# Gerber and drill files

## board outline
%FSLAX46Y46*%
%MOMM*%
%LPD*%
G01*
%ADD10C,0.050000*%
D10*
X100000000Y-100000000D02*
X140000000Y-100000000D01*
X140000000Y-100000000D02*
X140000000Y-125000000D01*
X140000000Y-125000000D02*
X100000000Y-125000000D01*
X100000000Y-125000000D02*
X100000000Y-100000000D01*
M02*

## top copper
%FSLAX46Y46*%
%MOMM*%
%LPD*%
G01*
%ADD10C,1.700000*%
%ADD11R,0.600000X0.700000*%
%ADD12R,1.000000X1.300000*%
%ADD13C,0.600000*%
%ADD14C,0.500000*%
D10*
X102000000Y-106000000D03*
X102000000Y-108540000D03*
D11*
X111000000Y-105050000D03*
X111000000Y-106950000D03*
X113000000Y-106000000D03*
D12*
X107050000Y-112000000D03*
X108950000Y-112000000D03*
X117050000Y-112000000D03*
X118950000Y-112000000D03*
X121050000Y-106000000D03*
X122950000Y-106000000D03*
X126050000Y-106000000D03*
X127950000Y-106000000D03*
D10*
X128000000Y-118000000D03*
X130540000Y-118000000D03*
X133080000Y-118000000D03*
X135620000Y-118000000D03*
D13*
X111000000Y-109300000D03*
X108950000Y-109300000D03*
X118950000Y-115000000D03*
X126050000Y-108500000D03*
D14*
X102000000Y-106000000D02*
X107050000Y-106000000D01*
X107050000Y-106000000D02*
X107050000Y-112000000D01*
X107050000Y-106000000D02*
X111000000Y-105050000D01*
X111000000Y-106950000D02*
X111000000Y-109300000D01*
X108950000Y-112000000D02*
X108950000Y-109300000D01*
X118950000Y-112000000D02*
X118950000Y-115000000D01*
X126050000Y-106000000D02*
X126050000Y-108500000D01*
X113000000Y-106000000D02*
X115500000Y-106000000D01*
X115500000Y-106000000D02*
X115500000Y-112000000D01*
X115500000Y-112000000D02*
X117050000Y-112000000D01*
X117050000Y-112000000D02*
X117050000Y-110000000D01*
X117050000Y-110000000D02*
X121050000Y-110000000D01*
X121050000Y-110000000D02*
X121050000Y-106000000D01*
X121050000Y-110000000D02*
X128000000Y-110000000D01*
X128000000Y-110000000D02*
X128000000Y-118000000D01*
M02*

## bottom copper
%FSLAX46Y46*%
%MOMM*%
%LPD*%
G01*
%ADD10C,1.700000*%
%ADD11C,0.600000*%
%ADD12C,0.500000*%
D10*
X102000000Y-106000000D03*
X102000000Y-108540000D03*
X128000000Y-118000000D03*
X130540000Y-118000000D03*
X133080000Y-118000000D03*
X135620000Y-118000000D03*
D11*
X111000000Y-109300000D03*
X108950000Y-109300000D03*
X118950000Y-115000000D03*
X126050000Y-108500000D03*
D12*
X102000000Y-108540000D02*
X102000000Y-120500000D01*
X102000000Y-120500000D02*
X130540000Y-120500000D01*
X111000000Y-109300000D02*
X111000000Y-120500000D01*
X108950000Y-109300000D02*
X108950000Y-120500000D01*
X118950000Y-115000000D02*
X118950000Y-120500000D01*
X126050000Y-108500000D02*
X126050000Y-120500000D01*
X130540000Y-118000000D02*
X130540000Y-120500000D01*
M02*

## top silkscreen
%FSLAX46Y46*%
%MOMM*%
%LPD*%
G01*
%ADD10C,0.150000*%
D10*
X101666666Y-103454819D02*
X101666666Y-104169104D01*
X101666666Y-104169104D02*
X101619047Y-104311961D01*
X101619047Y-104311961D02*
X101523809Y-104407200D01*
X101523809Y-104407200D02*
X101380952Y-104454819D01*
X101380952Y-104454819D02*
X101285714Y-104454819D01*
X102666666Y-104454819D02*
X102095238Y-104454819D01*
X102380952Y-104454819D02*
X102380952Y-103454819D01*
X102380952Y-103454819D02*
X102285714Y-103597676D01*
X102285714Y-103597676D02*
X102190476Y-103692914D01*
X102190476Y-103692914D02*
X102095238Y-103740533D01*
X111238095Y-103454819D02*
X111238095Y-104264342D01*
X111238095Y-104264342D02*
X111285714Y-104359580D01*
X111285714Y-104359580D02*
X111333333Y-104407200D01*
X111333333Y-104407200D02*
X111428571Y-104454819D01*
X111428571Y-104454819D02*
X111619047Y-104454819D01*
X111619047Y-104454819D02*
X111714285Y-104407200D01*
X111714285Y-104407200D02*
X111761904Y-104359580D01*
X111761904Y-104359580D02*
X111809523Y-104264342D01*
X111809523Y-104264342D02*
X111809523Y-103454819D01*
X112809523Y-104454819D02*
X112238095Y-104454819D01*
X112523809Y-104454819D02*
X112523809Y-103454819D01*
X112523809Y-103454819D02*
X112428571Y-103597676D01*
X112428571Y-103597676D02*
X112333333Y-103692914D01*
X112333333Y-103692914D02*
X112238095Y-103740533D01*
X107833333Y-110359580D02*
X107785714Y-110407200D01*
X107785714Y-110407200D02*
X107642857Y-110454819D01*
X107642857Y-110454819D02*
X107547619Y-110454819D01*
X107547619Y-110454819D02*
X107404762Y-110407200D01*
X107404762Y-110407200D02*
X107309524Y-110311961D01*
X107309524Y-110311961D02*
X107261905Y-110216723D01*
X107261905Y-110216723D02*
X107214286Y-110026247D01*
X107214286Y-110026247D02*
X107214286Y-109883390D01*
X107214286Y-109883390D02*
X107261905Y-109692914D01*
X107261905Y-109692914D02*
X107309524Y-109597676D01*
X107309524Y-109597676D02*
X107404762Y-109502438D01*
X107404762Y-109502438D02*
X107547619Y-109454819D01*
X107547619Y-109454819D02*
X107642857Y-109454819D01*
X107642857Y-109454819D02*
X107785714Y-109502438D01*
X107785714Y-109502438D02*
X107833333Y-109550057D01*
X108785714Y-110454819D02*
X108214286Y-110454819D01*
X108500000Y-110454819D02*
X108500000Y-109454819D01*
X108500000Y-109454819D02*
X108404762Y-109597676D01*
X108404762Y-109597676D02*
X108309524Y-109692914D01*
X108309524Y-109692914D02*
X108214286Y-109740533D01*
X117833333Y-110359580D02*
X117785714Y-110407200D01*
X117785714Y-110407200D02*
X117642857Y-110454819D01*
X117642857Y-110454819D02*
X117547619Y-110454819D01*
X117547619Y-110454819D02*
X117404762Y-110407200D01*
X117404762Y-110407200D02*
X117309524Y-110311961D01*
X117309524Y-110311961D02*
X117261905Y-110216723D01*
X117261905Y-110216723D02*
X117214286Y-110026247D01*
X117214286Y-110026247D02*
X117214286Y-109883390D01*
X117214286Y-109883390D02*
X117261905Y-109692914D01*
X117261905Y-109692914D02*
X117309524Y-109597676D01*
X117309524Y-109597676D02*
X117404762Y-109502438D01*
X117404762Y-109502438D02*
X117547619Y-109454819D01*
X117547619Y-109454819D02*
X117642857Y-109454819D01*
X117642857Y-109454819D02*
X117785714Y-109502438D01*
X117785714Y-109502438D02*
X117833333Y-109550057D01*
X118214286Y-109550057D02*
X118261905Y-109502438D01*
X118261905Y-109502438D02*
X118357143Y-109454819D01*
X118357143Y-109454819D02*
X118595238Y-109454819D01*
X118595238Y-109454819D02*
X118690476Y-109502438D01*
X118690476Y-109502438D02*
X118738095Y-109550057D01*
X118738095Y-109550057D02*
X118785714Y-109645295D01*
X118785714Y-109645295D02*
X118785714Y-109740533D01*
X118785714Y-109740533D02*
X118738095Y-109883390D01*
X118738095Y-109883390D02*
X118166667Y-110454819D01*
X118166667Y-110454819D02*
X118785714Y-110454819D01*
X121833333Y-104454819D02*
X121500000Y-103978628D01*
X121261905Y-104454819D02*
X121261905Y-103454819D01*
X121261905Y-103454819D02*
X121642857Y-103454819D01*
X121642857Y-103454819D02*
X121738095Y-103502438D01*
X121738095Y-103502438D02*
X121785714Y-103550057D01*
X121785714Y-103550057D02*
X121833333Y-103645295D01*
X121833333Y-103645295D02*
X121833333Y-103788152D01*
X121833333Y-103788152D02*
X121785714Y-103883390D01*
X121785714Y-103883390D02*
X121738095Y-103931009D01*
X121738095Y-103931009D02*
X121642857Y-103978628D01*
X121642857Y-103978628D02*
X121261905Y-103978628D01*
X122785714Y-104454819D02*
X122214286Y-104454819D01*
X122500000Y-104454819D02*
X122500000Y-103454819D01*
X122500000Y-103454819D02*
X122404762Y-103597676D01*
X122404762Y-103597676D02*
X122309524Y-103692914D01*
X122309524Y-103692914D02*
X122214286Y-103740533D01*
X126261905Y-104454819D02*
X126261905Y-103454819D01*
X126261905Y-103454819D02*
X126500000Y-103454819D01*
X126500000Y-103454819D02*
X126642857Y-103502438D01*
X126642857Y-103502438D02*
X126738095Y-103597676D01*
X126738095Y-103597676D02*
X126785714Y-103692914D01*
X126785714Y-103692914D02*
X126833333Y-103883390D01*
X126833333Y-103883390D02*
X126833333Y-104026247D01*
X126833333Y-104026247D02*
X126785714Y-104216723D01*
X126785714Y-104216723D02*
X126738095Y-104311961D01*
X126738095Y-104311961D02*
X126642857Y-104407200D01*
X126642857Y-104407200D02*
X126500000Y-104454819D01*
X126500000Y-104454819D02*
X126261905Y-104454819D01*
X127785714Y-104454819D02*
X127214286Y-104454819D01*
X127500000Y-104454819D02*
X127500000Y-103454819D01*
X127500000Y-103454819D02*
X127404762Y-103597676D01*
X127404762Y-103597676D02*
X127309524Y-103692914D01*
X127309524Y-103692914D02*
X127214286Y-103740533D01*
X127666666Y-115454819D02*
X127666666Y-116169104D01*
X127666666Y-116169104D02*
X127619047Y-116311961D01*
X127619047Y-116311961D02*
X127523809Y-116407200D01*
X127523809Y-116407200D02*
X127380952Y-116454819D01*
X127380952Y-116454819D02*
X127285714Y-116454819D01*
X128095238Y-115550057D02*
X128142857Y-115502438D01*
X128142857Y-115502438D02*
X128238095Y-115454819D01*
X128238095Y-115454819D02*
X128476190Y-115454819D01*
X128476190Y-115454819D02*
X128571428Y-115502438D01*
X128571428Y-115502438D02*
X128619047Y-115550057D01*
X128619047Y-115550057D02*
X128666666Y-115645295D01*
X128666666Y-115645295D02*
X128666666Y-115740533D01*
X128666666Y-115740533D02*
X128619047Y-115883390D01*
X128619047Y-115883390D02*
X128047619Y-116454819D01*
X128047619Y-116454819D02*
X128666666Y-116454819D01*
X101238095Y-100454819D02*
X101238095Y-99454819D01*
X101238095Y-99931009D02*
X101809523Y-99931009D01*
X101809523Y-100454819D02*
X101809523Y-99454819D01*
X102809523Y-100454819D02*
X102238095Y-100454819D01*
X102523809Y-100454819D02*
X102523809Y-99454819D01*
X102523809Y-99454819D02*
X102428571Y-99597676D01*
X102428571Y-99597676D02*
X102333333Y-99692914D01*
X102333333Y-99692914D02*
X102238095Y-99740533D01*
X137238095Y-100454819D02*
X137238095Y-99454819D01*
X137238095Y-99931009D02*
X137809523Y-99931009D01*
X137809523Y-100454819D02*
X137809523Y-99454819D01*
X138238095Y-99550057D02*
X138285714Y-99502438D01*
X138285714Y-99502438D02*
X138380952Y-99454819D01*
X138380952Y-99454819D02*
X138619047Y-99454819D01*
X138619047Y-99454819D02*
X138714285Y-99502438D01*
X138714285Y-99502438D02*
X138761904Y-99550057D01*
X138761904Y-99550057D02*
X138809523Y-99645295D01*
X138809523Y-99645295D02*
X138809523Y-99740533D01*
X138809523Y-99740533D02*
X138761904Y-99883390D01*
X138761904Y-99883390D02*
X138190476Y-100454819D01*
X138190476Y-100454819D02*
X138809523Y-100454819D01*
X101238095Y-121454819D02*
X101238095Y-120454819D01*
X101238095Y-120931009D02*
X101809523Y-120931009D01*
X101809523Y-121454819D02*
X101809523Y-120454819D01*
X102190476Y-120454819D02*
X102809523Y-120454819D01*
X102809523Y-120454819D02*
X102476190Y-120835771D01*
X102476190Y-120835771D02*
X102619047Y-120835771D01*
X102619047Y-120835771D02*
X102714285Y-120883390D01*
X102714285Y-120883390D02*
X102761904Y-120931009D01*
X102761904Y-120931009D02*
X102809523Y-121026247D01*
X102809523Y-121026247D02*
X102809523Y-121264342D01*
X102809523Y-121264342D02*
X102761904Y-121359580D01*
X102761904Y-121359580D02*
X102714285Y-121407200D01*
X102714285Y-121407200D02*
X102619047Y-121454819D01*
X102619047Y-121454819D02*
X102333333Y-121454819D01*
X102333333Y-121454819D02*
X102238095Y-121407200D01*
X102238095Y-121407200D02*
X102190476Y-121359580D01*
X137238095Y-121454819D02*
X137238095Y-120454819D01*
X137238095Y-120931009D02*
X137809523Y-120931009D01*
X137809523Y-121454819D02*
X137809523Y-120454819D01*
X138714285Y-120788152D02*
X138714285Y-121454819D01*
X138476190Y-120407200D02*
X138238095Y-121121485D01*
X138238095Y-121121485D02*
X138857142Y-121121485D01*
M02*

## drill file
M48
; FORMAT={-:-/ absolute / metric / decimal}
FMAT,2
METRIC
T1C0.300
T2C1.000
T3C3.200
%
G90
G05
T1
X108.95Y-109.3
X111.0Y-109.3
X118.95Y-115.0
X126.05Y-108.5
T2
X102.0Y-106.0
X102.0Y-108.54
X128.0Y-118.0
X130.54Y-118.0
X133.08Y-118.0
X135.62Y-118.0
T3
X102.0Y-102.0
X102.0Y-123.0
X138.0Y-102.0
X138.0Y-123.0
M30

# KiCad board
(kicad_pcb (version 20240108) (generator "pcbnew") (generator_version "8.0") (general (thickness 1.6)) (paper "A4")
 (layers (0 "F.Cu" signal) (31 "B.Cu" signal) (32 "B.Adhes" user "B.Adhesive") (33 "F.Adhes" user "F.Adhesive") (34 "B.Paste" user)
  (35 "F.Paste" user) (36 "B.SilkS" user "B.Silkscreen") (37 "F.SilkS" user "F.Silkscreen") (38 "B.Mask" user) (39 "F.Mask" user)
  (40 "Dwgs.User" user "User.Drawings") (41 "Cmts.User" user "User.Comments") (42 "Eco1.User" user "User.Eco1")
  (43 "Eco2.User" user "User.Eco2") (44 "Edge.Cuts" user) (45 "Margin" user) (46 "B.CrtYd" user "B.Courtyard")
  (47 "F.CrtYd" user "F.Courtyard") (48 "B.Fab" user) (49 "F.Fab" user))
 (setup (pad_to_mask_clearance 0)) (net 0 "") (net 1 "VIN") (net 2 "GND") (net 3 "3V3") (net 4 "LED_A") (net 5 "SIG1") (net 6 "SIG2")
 (gr_line (start 100 100) (end 140 100) (stroke (width 0.05) (type default)) (layer "Edge.Cuts"))
 (gr_line (start 140 100) (end 140 125) (stroke (width 0.05) (type default)) (layer "Edge.Cuts"))
 (gr_line (start 140 125) (end 100 125) (stroke (width 0.05) (type default)) (layer "Edge.Cuts"))
 (gr_line (start 100 125) (end 100 100) (stroke (width 0.05) (type default)) (layer "Edge.Cuts"))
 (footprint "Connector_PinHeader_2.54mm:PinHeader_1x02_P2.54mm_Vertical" (layer "F.Cu") (at 102 106)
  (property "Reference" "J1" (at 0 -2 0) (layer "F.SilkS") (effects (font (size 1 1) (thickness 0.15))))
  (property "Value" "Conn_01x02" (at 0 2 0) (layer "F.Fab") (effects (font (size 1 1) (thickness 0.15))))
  (pad "1" thru_hole circle (at 0 0) (size 1.7 1.7) (drill 1) (layers "*.Cu" "*.Mask") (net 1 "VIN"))
  (pad "2" thru_hole circle (at 0 2.54) (size 1.7 1.7) (drill 1) (layers "*.Cu" "*.Mask") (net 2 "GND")))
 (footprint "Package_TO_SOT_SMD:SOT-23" (layer "F.Cu") (at 112 106)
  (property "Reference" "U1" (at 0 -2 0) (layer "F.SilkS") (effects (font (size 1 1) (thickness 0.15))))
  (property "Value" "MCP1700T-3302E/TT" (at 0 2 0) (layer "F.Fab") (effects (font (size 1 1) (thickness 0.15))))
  (pad "1" smd rect (at -1 -0.95) (size 0.6 0.7) (layers "F.Cu" "F.Paste" "F.Mask") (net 1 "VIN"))
  (pad "2" smd rect (at -1 0.95) (size 0.6 0.7) (layers "F.Cu" "F.Paste" "F.Mask") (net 2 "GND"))
  (pad "3" smd rect (at 1 0) (size 0.6 0.7) (layers "F.Cu" "F.Paste" "F.Mask") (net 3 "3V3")))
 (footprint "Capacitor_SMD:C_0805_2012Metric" (layer "F.Cu") (at 108 112)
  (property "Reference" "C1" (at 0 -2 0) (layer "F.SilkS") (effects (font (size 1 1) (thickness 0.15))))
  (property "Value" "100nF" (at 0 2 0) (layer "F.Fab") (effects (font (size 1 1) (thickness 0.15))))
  (pad "1" smd rect (at -0.95 0) (size 1 1.3) (layers "F.Cu" "F.Paste" "F.Mask") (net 1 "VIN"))
  (pad "2" smd rect (at 0.95 0) (size 1 1.3) (layers "F.Cu" "F.Paste" "F.Mask") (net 2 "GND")))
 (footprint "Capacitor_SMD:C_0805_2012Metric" (layer "F.Cu") (at 118 112)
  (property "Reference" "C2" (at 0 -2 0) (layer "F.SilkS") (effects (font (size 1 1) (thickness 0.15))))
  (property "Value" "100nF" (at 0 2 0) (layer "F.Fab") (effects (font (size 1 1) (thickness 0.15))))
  (pad "1" smd rect (at -0.95 0) (size 1 1.3) (layers "F.Cu" "F.Paste" "F.Mask") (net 3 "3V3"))
  (pad "2" smd rect (at 0.95 0) (size 1 1.3) (layers "F.Cu" "F.Paste" "F.Mask") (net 2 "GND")))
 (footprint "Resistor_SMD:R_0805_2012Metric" (layer "F.Cu") (at 122 106)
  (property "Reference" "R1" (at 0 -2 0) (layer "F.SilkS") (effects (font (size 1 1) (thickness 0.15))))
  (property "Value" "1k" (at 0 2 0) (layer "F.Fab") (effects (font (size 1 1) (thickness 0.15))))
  (pad "1" smd rect (at -0.95 0) (size 1 1.3) (layers "F.Cu" "F.Paste" "F.Mask") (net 3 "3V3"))
  (pad "2" smd rect (at 0.95 0) (size 1 1.3) (layers "F.Cu" "F.Paste" "F.Mask") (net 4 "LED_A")))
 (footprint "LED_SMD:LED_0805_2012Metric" (layer "F.Cu") (at 127 106)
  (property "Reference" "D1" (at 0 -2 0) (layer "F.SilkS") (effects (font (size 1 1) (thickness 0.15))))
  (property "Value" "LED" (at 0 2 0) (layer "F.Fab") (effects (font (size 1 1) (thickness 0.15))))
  (pad "1" smd rect (at -0.95 0) (size 1 1.3) (layers "F.Cu" "F.Paste" "F.Mask") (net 2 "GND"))
  (pad "2" smd rect (at 0.95 0) (size 1 1.3) (layers "F.Cu" "F.Paste" "F.Mask") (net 4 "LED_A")))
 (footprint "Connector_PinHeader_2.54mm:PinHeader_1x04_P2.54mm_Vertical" (layer "F.Cu") (at 128 118)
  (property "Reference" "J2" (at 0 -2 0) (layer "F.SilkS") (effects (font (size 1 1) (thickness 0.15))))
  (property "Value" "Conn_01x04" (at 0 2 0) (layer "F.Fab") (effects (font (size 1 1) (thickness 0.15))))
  (pad "1" thru_hole circle (at 0 0) (size 1.7 1.7) (drill 1) (layers "*.Cu" "*.Mask") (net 3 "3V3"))
  (pad "2" thru_hole circle (at 2.54 0) (size 1.7 1.7) (drill 1) (layers "*.Cu" "*.Mask") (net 2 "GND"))
  (pad "3" thru_hole circle (at 5.08 0) (size 1.7 1.7) (drill 1) (layers "*.Cu" "*.Mask") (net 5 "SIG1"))
  (pad "4" thru_hole circle (at 7.62 0) (size 1.7 1.7) (drill 1) (layers "*.Cu" "*.Mask") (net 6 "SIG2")))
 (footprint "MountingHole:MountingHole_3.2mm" (layer "F.Cu") (at 102 102)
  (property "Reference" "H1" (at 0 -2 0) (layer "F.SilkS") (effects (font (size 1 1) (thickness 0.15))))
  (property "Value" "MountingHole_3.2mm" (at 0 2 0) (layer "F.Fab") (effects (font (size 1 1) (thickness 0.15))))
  (pad "1" np_thru_hole circle (at 0 0) (size 3.2 3.2) (drill 3.2) (layers "*.Cu" "*.Mask")))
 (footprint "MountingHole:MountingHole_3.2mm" (layer "F.Cu") (at 138 102)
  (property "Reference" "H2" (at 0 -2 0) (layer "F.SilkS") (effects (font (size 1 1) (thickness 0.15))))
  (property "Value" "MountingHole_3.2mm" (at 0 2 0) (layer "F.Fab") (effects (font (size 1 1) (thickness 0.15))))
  (pad "1" np_thru_hole circle (at 0 0) (size 3.2 3.2) (drill 3.2) (layers "*.Cu" "*.Mask")))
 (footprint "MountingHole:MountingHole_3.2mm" (layer "F.Cu") (at 102 123)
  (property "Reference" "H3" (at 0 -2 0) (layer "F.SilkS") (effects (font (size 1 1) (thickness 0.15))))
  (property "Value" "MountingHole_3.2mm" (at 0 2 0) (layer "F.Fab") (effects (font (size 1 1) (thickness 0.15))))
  (pad "1" np_thru_hole circle (at 0 0) (size 3.2 3.2) (drill 3.2) (layers "*.Cu" "*.Mask")))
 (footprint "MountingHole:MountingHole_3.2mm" (layer "F.Cu") (at 138 123)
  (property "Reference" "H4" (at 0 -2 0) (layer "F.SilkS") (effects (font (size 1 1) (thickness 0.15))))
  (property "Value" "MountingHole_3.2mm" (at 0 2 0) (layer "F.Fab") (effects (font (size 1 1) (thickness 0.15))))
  (pad "1" np_thru_hole circle (at 0 0) (size 3.2 3.2) (drill 3.2) (layers "*.Cu" "*.Mask")))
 (segment (start 102 106) (end 107.05 106) (width 0.5) (layer "F.Cu") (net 1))
 (segment (start 107.05 106) (end 107.05 112) (width 0.5) (layer "F.Cu") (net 1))
 (segment (start 107.05 106) (end 111 105.05) (width 0.5) (layer "F.Cu") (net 1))
 (segment (start 111 106.95) (end 111 109.3) (width 0.5) (layer "F.Cu") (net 2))
 (segment (start 108.95 112) (end 108.95 109.3) (width 0.5) (layer "F.Cu") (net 2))
 (segment (start 118.95 112) (end 118.95 115) (width 0.5) (layer "F.Cu") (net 2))
 (segment (start 126.05 106) (end 126.05 108.5) (width 0.5) (layer "F.Cu") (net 2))
 (segment (start 113 106) (end 115.5 106) (width 0.5) (layer "F.Cu") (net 3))
 (segment (start 115.5 106) (end 115.5 112) (width 0.5) (layer "F.Cu") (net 3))
 (segment (start 115.5 112) (end 117.05 112) (width 0.5) (layer "F.Cu") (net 3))
 (segment (start 117.05 112) (end 117.05 110) (width 0.5) (layer "F.Cu") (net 3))
 (segment (start 117.05 110) (end 121.05 110) (width 0.5) (layer "F.Cu") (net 3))
 (segment (start 121.05 110) (end 121.05 106) (width 0.5) (layer "F.Cu") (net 3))
 (segment (start 121.05 110) (end 128 110) (width 0.5) (layer "F.Cu") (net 3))
 (segment (start 128 110) (end 128 118) (width 0.5) (layer "F.Cu") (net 3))
 (segment (start 102 108.54) (end 102 120.5) (width 0.5) (layer "B.Cu") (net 2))
 (segment (start 102 120.5) (end 130.54 120.5) (width 0.5) (layer "B.Cu") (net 2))
 (segment (start 111 109.3) (end 111 120.5) (width 0.5) (layer "B.Cu") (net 2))
 (segment (start 108.95 109.3) (end 108.95 120.5) (width 0.5) (layer "B.Cu") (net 2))
 (segment (start 118.95 115) (end 118.95 120.5) (width 0.5) (layer "B.Cu") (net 2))
 (segment (start 126.05 108.5) (end 126.05 120.5) (width 0.5) (layer "B.Cu") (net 2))
 (segment (start 130.54 118) (end 130.54 120.5) (width 0.5) (layer "B.Cu") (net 2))
 (via (at 111 109.3) (size 0.6) (drill 0.3) (layers "F.Cu" "B.Cu") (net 2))
 (via (at 108.95 109.3) (size 0.6) (drill 0.3) (layers "F.Cu" "B.Cu") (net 2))
 (via (at 118.95 115) (size 0.6) (drill 0.3) (layers "F.Cu" "B.Cu") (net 2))
 (via (at 126.05 108.5) (size 0.6) (drill 0.3) (layers "F.Cu" "B.Cu") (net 2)))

